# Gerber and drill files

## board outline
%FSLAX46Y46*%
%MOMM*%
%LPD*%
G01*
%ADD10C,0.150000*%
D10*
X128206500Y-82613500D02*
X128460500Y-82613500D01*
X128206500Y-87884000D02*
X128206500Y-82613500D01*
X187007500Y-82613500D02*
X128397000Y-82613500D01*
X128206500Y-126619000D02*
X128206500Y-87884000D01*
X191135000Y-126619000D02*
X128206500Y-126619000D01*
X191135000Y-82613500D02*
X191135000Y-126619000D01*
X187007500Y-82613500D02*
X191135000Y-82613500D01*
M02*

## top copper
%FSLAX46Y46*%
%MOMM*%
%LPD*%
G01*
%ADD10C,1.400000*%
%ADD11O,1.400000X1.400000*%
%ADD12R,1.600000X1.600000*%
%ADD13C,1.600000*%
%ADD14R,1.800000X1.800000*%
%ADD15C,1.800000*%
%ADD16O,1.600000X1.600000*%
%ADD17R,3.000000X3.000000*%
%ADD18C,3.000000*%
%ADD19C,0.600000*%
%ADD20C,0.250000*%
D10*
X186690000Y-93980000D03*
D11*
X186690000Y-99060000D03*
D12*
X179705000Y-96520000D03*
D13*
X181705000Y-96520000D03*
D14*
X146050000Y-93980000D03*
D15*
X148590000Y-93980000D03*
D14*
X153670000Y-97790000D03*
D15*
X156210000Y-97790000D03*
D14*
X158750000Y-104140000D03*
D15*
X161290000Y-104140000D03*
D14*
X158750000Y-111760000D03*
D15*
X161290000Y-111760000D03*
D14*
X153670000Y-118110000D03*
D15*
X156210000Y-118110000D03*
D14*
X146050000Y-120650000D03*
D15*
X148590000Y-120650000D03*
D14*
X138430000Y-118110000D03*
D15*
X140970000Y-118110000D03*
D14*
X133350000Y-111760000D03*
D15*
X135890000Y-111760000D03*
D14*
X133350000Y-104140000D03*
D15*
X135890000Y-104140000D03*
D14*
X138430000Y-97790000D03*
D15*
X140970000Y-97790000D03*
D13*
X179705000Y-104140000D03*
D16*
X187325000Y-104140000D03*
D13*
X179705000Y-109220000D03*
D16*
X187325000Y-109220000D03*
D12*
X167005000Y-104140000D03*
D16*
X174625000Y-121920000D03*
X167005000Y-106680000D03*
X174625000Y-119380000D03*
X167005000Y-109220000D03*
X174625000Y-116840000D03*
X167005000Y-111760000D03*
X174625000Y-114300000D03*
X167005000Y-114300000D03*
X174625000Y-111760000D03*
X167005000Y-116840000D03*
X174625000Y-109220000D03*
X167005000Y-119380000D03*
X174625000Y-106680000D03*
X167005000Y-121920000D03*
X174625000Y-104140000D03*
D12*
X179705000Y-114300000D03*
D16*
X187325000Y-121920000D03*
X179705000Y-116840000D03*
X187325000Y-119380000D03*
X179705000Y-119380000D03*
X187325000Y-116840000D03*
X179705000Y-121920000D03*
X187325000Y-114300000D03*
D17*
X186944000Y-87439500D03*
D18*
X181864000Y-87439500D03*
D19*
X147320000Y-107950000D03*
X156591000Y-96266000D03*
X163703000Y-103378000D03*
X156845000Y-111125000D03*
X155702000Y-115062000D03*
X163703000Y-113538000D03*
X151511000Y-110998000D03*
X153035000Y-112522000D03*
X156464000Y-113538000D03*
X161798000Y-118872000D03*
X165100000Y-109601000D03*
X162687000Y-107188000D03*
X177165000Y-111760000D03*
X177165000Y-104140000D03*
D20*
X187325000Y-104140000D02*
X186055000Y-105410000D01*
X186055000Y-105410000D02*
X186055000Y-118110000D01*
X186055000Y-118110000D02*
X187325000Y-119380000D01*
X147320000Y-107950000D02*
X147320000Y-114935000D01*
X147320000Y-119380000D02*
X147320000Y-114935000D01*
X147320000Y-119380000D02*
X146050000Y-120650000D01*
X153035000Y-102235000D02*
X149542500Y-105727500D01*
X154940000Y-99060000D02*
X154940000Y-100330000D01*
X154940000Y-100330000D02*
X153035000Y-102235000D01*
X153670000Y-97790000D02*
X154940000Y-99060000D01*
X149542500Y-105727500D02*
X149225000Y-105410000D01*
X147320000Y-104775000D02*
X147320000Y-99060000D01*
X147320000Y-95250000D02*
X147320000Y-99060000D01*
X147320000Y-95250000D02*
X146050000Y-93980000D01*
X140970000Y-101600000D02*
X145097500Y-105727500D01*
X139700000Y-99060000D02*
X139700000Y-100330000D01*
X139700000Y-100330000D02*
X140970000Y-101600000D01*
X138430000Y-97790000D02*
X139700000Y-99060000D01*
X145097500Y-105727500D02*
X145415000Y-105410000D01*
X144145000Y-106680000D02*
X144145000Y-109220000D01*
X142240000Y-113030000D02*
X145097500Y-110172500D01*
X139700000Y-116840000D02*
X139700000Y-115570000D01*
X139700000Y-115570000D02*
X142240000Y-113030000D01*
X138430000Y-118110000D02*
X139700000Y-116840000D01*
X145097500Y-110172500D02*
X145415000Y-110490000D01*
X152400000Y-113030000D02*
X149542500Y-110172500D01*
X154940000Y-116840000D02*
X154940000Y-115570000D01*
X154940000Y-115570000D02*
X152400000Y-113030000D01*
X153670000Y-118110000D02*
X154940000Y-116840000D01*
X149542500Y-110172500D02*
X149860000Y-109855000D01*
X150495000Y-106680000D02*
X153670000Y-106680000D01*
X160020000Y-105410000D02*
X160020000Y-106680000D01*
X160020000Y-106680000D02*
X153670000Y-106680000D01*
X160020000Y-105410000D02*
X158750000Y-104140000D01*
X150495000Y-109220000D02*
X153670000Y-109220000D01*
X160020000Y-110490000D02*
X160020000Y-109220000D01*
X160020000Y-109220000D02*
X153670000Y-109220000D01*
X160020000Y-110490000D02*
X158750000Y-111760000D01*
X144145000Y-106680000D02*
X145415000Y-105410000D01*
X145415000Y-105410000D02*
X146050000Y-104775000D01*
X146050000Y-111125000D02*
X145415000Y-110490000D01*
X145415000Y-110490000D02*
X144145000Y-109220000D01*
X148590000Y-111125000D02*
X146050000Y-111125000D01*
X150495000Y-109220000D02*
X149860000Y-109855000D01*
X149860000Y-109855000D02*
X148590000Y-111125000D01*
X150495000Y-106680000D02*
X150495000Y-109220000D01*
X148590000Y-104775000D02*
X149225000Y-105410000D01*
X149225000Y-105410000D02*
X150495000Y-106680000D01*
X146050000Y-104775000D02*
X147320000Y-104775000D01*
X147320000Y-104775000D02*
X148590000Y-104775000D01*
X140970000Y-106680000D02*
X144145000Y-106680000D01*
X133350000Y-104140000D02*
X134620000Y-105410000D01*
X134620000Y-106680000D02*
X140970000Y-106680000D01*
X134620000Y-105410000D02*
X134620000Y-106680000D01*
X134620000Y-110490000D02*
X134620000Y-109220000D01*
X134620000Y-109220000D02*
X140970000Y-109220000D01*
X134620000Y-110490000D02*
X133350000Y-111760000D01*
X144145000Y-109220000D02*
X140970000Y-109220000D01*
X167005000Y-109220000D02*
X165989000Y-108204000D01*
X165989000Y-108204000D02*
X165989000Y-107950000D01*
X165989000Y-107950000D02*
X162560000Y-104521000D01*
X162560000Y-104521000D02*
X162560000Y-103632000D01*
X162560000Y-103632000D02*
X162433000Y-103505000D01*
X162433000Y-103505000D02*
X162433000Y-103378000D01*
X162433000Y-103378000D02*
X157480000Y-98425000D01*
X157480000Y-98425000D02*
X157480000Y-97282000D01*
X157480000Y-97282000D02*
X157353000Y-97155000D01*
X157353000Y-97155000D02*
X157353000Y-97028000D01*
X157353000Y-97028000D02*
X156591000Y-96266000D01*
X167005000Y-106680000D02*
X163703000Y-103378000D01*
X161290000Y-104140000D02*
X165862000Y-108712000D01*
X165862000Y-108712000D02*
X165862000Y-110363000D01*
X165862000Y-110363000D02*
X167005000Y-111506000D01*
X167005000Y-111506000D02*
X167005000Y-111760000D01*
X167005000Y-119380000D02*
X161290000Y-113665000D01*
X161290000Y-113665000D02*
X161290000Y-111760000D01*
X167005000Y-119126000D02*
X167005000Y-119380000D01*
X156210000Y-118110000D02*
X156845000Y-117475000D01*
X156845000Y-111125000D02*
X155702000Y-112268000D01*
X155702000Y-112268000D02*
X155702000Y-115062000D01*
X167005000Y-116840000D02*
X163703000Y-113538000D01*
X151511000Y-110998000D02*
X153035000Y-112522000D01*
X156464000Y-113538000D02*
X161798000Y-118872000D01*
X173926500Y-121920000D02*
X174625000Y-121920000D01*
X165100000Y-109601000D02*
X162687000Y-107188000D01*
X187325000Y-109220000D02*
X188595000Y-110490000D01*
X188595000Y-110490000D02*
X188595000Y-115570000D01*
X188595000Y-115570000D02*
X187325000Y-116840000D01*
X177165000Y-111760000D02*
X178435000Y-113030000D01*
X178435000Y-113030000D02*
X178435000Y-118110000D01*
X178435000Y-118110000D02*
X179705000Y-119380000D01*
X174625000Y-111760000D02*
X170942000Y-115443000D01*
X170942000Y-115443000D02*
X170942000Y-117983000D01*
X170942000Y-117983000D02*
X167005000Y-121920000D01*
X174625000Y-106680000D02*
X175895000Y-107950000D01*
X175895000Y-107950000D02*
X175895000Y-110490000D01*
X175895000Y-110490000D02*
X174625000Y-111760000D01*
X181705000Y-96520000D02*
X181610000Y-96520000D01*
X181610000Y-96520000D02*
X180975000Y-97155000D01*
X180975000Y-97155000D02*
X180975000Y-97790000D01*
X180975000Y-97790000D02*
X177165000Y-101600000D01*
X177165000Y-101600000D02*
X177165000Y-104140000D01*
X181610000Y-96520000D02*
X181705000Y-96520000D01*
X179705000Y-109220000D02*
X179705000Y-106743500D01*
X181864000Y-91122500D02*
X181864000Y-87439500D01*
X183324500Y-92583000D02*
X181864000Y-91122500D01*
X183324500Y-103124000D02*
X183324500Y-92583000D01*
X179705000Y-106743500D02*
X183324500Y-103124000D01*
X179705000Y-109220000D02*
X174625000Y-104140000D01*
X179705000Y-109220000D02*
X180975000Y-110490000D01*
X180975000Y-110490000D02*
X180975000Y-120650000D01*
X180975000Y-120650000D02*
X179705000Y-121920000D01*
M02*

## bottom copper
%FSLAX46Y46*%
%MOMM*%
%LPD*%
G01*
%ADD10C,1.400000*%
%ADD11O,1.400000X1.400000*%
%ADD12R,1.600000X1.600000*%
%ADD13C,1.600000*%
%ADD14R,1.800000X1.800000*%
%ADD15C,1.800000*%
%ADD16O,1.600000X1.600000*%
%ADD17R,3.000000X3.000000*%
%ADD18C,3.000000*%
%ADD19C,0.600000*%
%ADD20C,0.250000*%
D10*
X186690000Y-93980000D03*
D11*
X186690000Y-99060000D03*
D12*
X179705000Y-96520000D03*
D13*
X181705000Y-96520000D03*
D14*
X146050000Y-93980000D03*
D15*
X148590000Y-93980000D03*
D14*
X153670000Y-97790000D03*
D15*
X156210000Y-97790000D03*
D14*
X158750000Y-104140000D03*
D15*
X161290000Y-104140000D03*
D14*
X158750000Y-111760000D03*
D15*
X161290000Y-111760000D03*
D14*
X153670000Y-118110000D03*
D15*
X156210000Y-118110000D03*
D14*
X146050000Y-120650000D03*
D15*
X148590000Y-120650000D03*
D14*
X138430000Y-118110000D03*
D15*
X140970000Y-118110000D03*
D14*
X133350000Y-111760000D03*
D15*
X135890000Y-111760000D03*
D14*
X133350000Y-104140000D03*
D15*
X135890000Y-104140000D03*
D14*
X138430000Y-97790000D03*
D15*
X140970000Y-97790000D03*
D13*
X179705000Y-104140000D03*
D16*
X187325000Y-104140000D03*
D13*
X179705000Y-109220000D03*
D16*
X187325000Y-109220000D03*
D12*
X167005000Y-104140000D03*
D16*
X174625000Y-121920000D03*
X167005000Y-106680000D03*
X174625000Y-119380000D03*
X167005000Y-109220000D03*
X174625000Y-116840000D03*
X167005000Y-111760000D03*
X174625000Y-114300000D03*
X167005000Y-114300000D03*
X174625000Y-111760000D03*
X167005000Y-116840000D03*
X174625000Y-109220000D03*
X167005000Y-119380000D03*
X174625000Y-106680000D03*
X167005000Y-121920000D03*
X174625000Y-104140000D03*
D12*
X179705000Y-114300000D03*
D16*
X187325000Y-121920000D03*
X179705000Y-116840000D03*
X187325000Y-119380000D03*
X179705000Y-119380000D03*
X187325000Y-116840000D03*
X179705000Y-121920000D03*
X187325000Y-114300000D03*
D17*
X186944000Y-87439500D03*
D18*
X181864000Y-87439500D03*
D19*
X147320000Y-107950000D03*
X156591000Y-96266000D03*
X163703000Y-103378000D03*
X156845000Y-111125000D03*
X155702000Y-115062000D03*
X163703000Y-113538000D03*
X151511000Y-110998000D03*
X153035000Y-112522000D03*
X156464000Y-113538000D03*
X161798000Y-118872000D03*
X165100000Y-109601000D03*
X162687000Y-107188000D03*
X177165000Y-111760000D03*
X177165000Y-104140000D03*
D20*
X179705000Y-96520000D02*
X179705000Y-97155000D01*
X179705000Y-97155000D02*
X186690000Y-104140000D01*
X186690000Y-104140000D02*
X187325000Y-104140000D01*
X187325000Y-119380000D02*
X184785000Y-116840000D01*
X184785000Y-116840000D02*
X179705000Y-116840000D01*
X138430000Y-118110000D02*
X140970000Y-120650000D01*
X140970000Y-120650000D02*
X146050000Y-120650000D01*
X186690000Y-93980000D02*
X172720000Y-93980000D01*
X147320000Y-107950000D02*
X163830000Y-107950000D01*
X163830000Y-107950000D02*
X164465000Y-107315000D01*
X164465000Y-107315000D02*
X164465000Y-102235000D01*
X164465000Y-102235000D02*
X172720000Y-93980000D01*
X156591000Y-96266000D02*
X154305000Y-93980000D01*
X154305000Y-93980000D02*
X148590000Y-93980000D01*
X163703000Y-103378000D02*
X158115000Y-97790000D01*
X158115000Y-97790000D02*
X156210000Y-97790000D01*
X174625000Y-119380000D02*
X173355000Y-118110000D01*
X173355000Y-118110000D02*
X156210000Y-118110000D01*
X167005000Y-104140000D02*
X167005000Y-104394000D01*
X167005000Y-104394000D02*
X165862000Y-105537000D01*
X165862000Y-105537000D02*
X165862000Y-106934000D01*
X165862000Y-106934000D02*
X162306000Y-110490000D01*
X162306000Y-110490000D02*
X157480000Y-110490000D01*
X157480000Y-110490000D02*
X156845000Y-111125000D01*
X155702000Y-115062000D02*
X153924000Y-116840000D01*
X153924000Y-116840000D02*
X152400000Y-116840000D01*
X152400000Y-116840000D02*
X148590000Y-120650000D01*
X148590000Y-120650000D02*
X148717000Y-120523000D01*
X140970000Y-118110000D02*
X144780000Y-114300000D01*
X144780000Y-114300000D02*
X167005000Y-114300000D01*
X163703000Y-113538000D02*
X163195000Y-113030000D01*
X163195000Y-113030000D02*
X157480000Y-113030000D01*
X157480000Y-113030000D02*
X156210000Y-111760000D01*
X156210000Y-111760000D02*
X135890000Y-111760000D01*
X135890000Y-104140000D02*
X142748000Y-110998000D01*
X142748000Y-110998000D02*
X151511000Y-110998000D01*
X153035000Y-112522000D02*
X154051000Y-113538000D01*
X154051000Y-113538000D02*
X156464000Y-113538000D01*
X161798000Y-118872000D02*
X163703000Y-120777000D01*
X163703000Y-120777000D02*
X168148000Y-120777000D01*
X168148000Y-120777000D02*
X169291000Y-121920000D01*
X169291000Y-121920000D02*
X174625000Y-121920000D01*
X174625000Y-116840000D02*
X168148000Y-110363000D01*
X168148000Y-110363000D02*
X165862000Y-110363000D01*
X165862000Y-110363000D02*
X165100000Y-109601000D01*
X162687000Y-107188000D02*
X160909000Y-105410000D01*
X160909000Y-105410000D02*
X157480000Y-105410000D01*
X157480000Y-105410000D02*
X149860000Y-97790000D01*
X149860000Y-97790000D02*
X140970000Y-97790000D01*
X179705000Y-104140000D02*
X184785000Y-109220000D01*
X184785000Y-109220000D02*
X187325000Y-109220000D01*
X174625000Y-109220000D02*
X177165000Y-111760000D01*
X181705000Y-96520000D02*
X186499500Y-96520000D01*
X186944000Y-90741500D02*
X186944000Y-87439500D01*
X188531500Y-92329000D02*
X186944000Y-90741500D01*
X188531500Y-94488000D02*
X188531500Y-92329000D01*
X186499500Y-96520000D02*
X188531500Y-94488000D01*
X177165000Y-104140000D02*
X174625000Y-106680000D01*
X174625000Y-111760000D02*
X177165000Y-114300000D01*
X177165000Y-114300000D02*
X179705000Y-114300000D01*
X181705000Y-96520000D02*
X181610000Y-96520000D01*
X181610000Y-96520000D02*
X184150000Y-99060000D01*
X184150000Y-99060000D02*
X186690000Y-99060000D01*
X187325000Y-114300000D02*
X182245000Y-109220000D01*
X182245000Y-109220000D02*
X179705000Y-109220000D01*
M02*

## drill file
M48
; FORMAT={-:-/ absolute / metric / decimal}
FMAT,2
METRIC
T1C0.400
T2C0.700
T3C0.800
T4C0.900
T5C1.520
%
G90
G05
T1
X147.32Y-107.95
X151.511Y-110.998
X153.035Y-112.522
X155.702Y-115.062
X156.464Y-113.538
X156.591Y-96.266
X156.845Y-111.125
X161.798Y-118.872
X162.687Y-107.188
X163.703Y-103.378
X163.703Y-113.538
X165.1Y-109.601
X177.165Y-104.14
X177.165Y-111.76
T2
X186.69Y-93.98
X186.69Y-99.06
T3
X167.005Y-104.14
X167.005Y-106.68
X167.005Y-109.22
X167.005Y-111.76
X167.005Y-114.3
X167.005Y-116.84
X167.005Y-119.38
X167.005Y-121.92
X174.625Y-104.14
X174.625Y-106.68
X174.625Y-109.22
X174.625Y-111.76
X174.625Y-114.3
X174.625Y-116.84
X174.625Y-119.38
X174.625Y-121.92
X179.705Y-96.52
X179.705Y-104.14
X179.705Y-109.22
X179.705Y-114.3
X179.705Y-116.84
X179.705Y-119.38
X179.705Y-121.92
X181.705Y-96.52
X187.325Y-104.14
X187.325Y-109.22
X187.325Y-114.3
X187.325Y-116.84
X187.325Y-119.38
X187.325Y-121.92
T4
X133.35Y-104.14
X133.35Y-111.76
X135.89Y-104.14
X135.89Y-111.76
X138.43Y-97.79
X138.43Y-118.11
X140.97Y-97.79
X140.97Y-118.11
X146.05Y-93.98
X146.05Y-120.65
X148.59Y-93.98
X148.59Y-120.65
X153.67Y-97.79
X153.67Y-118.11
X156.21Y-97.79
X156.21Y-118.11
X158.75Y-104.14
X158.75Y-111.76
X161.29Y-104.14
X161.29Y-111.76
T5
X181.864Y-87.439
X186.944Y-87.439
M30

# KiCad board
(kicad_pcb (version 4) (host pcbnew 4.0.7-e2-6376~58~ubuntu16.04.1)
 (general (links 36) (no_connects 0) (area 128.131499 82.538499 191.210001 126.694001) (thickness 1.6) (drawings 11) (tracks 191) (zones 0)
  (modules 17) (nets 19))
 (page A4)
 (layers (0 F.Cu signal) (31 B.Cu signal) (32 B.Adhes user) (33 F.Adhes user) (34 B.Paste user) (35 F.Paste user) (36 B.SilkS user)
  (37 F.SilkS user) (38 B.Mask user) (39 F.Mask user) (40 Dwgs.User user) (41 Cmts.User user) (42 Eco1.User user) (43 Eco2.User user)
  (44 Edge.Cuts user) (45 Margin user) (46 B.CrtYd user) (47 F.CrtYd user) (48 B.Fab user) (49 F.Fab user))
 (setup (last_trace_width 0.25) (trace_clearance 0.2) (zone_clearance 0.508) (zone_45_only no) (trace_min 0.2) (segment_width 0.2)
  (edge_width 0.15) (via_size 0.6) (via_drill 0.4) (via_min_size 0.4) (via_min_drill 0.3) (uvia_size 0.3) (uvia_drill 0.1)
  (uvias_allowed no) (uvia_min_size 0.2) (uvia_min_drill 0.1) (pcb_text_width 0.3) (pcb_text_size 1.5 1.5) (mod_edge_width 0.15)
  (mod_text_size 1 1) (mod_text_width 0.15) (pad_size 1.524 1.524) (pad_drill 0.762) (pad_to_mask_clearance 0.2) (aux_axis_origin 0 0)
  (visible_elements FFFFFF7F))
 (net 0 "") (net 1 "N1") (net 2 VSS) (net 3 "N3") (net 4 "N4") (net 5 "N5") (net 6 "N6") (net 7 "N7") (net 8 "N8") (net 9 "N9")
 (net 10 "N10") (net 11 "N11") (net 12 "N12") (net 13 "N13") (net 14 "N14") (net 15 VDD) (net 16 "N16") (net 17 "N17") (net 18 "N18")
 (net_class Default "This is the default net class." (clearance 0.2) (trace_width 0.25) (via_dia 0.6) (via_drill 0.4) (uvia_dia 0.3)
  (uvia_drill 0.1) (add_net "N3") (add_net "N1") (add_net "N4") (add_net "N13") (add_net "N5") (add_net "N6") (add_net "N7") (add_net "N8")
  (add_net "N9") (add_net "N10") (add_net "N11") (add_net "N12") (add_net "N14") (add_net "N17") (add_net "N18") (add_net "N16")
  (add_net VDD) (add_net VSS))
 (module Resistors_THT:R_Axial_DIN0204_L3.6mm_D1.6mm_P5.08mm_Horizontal (layer F.Cu) (at 186.69 93.98 270)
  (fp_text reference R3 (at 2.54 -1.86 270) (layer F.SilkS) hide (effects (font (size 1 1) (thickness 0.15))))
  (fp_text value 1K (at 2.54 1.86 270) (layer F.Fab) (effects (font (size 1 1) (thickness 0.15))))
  (pad 1 thru_hole circle (at 0 0 270) (size 1.4 1.4) (drill 0.7) (layers *.Cu *.Mask) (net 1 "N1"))
  (pad 2 thru_hole oval (at 5.08 0 270) (size 1.4 1.4) (drill 0.7) (layers *.Cu *.Mask) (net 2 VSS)))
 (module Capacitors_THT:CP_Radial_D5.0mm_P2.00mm (layer F.Cu) (at 179.705 96.52)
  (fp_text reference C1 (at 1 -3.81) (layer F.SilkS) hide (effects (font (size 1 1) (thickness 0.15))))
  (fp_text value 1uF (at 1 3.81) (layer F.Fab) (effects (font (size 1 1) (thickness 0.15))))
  (pad 1 thru_hole rect (at 0 0) (size 1.6 1.6) (drill 0.8) (layers *.Cu *.Mask) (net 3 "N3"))
  (pad 2 thru_hole circle (at 2 0) (size 1.6 1.6) (drill 0.8) (layers *.Cu *.Mask) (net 2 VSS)))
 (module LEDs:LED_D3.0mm (layer F.Cu) (at 146.05 93.98)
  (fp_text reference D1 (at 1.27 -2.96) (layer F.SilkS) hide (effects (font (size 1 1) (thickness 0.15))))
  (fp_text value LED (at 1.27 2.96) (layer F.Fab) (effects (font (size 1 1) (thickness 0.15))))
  (pad 1 thru_hole rect (at 0 0) (size 1.8 1.8) (drill 0.9) (layers *.Cu *.Mask) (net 1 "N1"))
  (pad 2 thru_hole circle (at 2.54 0) (size 1.8 1.8) (drill 0.9) (layers *.Cu *.Mask) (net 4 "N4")))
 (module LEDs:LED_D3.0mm (layer F.Cu) (at 153.67 97.79)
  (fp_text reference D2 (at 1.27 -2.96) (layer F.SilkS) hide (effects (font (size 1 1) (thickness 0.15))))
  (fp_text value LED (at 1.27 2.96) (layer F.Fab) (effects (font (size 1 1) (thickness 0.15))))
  (pad 1 thru_hole rect (at 0 0) (size 1.8 1.8) (drill 0.9) (layers *.Cu *.Mask) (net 1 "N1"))
  (pad 2 thru_hole circle (at 2.54 0) (size 1.8 1.8) (drill 0.9) (layers *.Cu *.Mask) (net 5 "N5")))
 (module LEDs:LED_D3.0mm (layer F.Cu) (at 158.75 104.14)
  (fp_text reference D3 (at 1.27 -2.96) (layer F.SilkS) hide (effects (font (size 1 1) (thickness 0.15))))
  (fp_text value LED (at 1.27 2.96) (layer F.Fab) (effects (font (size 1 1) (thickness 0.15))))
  (pad 1 thru_hole rect (at 0 0) (size 1.8 1.8) (drill 0.9) (layers *.Cu *.Mask) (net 1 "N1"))
  (pad 2 thru_hole circle (at 2.54 0) (size 1.8 1.8) (drill 0.9) (layers *.Cu *.Mask) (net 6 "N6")))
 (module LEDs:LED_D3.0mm (layer F.Cu) (at 158.75 111.76)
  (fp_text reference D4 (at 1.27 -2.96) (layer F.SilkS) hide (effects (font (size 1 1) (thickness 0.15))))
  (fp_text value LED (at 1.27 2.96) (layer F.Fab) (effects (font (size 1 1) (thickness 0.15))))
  (pad 1 thru_hole rect (at 0 0) (size 1.8 1.8) (drill 0.9) (layers *.Cu *.Mask) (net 1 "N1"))
  (pad 2 thru_hole circle (at 2.54 0) (size 1.8 1.8) (drill 0.9) (layers *.Cu *.Mask) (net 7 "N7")))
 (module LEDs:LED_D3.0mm (layer F.Cu) (at 153.67 118.11)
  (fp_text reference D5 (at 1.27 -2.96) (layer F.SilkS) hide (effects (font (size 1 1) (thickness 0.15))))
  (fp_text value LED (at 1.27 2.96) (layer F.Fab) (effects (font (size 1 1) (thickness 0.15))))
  (pad 1 thru_hole rect (at 0 0) (size 1.8 1.8) (drill 0.9) (layers *.Cu *.Mask) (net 1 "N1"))
  (pad 2 thru_hole circle (at 2.54 0) (size 1.8 1.8) (drill 0.9) (layers *.Cu *.Mask) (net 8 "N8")))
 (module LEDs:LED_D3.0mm (layer F.Cu) (at 146.05 120.65)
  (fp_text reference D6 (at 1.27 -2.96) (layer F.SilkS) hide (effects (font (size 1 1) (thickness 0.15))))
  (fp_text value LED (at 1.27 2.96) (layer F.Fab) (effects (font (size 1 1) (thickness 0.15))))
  (pad 1 thru_hole rect (at 0 0) (size 1.8 1.8) (drill 0.9) (layers *.Cu *.Mask) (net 1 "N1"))
  (pad 2 thru_hole circle (at 2.54 0) (size 1.8 1.8) (drill 0.9) (layers *.Cu *.Mask) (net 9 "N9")))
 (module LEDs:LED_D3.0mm (layer F.Cu) (at 138.43 118.11)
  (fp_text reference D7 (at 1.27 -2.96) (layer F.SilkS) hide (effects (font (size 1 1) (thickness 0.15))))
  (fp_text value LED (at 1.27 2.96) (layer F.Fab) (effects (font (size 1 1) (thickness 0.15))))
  (pad 1 thru_hole rect (at 0 0) (size 1.8 1.8) (drill 0.9) (layers *.Cu *.Mask) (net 1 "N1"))
  (pad 2 thru_hole circle (at 2.54 0) (size 1.8 1.8) (drill 0.9) (layers *.Cu *.Mask) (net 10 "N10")))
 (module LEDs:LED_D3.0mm (layer F.Cu) (at 133.35 111.76)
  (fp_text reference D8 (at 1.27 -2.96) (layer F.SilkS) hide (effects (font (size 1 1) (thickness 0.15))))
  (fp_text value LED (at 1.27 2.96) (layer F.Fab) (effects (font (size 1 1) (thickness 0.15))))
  (pad 1 thru_hole rect (at 0 0) (size 1.8 1.8) (drill 0.9) (layers *.Cu *.Mask) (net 1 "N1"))
  (pad 2 thru_hole circle (at 2.54 0) (size 1.8 1.8) (drill 0.9) (layers *.Cu *.Mask) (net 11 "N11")))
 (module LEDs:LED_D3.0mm (layer F.Cu) (at 133.35 104.14)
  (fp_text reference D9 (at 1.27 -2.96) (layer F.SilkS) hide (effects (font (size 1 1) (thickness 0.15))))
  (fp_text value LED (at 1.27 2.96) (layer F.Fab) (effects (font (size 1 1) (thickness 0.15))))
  (pad 1 thru_hole rect (at 0 0) (size 1.8 1.8) (drill 0.9) (layers *.Cu *.Mask) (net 1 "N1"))
  (pad 2 thru_hole circle (at 2.54 0) (size 1.8 1.8) (drill 0.9) (layers *.Cu *.Mask) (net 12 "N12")))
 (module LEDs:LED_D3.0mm (layer F.Cu) (at 138.43 97.79)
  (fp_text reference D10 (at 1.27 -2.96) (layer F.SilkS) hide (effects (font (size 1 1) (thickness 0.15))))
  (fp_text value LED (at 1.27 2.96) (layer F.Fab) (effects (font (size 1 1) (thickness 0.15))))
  (pad 1 thru_hole rect (at 0 0) (size 1.8 1.8) (drill 0.9) (layers *.Cu *.Mask) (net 1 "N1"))
  (pad 2 thru_hole circle (at 2.54 0) (size 1.8 1.8) (drill 0.9) (layers *.Cu *.Mask) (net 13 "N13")))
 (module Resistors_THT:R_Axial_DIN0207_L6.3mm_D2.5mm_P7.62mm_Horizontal (layer F.Cu) (at 179.705 104.14)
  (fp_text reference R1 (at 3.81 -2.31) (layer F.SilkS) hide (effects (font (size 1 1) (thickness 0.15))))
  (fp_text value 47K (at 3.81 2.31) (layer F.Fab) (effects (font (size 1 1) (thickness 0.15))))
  (pad 1 thru_hole circle (at 0 0) (size 1.6 1.6) (drill 0.8) (layers *.Cu *.Mask) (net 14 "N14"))
  (pad 2 thru_hole oval (at 7.62 0) (size 1.6 1.6) (drill 0.8) (layers *.Cu *.Mask) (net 3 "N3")))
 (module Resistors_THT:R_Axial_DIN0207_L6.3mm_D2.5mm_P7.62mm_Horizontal (layer F.Cu) (at 179.705 109.22)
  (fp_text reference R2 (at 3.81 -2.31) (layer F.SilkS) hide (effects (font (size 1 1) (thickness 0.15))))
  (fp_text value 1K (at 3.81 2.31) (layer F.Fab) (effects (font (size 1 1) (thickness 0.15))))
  (pad 1 thru_hole circle (at 0 0) (size 1.6 1.6) (drill 0.8) (layers *.Cu *.Mask) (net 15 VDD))
  (pad 2 thru_hole oval (at 7.62 0) (size 1.6 1.6) (drill 0.8) (layers *.Cu *.Mask) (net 14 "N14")))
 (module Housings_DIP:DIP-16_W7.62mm (layer F.Cu) (at 167.005 104.14)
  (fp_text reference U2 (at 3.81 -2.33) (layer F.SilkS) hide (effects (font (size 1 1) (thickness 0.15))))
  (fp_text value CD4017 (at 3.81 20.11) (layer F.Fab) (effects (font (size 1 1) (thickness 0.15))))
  (pad 1 thru_hole rect (at 0 0) (size 1.6 1.6) (drill 0.8) (layers *.Cu *.Mask) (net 9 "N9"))
  (pad 9 thru_hole oval (at 7.62 17.78) (size 1.6 1.6) (drill 0.8) (layers *.Cu *.Mask) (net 12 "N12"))
  (pad 2 thru_hole oval (at 0 2.54) (size 1.6 1.6) (drill 0.8) (layers *.Cu *.Mask) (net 5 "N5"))
  (pad 10 thru_hole oval (at 7.62 15.24) (size 1.6 1.6) (drill 0.8) (layers *.Cu *.Mask) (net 8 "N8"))
  (pad 3 thru_hole oval (at 0 5.08) (size 1.6 1.6) (drill 0.8) (layers *.Cu *.Mask) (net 4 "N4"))
  (pad 11 thru_hole oval (at 7.62 12.7) (size 1.6 1.6) (drill 0.8) (layers *.Cu *.Mask) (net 13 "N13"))
  (pad 4 thru_hole oval (at 0 7.62) (size 1.6 1.6) (drill 0.8) (layers *.Cu *.Mask) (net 6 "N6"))
  (pad 12 thru_hole oval (at 7.62 10.16) (size 1.6 1.6) (drill 0.8) (layers *.Cu *.Mask) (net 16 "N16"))
  (pad 5 thru_hole oval (at 0 10.16) (size 1.6 1.6) (drill 0.8) (layers *.Cu *.Mask) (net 10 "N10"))
  (pad 13 thru_hole oval (at 7.62 7.62) (size 1.6 1.6) (drill 0.8) (layers *.Cu *.Mask) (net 2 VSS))
  (pad 6 thru_hole oval (at 0 12.7) (size 1.6 1.6) (drill 0.8) (layers *.Cu *.Mask) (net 11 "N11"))
  (pad 14 thru_hole oval (at 7.62 5.08) (size 1.6 1.6) (drill 0.8) (layers *.Cu *.Mask) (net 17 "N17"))
  (pad 7 thru_hole oval (at 0 15.24) (size 1.6 1.6) (drill 0.8) (layers *.Cu *.Mask) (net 7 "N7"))
  (pad 15 thru_hole oval (at 7.62 2.54) (size 1.6 1.6) (drill 0.8) (layers *.Cu *.Mask) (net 2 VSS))
  (pad 8 thru_hole oval (at 0 17.78) (size 1.6 1.6) (drill 0.8) (layers *.Cu *.Mask) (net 2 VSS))
  (pad 16 thru_hole oval (at 7.62 0) (size 1.6 1.6) (drill 0.8) (layers *.Cu *.Mask) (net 15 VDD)))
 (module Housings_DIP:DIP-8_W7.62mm (layer F.Cu) (at 179.705 114.3)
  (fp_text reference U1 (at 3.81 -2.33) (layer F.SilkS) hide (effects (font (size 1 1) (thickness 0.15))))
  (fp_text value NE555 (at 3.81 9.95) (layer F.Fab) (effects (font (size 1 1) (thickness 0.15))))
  (pad 1 thru_hole rect (at 0 0) (size 1.6 1.6) (drill 0.8) (layers *.Cu *.Mask) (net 2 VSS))
  (pad 5 thru_hole oval (at 7.62 7.62) (size 1.6 1.6) (drill 0.8) (layers *.Cu *.Mask) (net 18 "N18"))
  (pad 2 thru_hole oval (at 0 2.54) (size 1.6 1.6) (drill 0.8) (layers *.Cu *.Mask) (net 3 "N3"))
  (pad 6 thru_hole oval (at 7.62 5.08) (size 1.6 1.6) (drill 0.8) (layers *.Cu *.Mask) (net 3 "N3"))
  (pad 3 thru_hole oval (at 0 5.08) (size 1.6 1.6) (drill 0.8) (layers *.Cu *.Mask) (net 17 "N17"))
  (pad 7 thru_hole oval (at 7.62 2.54) (size 1.6 1.6) (drill 0.8) (layers *.Cu *.Mask) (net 14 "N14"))
  (pad 4 thru_hole oval (at 0 7.62) (size 1.6 1.6) (drill 0.8) (layers *.Cu *.Mask) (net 15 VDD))
  (pad 8 thru_hole oval (at 7.62 0) (size 1.6 1.6) (drill 0.8) (layers *.Cu *.Mask) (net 15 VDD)))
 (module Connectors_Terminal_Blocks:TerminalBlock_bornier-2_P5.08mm (layer F.Cu) (at 186.944 87.4395 180)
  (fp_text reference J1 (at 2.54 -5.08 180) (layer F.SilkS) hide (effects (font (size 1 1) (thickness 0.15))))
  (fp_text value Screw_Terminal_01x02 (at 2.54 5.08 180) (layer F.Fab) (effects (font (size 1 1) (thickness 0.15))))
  (pad 1 thru_hole rect (at 0 0 180) (size 3 3) (drill 1.52) (layers *.Cu *.Mask) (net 2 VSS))
  (pad 2 thru_hole circle (at 5.08 0 180) (size 3 3) (drill 1.52) (layers *.Cu *.Mask) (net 15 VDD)))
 (gr_line (start 128.2065 82.6135) (end 128.4605 82.6135) (angle 90) (layer Edge.Cuts) (width 0.15))
 (gr_line (start 128.2065 87.884) (end 128.2065 82.6135) (angle 90) (layer Edge.Cuts) (width 0.15))
 (gr_line (start 187.0075 82.6135) (end 128.397 82.6135) (angle 90) (layer Edge.Cuts) (width 0.15))
 (gr_line (start 128.2065 126.619) (end 128.2065 87.884) (angle 90) (layer Edge.Cuts) (width 0.15))
 (gr_line (start 191.135 126.619) (end 128.2065 126.619) (angle 90) (layer Edge.Cuts) (width 0.15))
 (gr_line (start 191.135 82.6135) (end 191.135 126.619) (angle 90) (layer Edge.Cuts) (width 0.15))
 (gr_line (start 187.0075 82.6135) (end 191.135 82.6135) (angle 90) (layer Edge.Cuts) (width 0.15))
 (segment (start 179.705 96.52) (end 179.705 97.155) (width 0.25) (layer B.Cu) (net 3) (status 80000))
 (segment (start 179.705 97.155) (end 186.69 104.14) (width 0.25) (layer B.Cu) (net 3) (status 80000))
 (segment (start 186.69 104.14) (end 187.325 104.14) (width 0.25) (layer B.Cu) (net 3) (status 80000))
 (segment (start 187.325 119.38) (end 184.785 116.84) (width 0.25) (layer B.Cu) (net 3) (status 80000))
 (segment (start 184.785 116.84) (end 179.705 116.84) (width 0.25) (layer B.Cu) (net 3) (status 80000))
 (segment (start 187.325 104.14) (end 186.055 105.41) (width 0.25) (layer F.Cu) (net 3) (status 80000))
 (segment (start 186.055 105.41) (end 186.055 118.11) (width 0.25) (layer F.Cu) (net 3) (status 80000))
 (segment (start 186.055 118.11) (end 187.325 119.38) (width 0.25) (layer F.Cu) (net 3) (status 80000))
 (segment (start 138.43 118.11) (end 140.97 120.65) (width 0.25) (layer B.Cu) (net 1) (status 80000))
 (segment (start 140.97 120.65) (end 146.05 120.65) (width 0.25) (layer B.Cu) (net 1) (status 80000))
 (segment (start 186.69 93.98) (end 172.72 93.98) (width 0.25) (layer B.Cu) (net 1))
 (segment (start 147.32 107.95) (end 163.83 107.95) (width 0.25) (layer B.Cu) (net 1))
 (segment (start 163.83 107.95) (end 164.465 107.315) (width 0.25) (layer B.Cu) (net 1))
 (segment (start 164.465 107.315) (end 164.465 102.235) (width 0.25) (layer B.Cu) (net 1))
 (segment (start 164.465 102.235) (end 172.72 93.98) (width 0.25) (layer B.Cu) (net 1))
 (segment (start 147.32 107.95) (end 147.32 114.935) (width 0.25) (layer F.Cu) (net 1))
 (segment (start 147.32 119.38) (end 147.32 114.935) (width 0.25) (layer F.Cu) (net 1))
 (segment (start 147.32 119.38) (end 146.05 120.65) (width 0.25) (layer F.Cu) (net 1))
 (via (at 147.32 107.95) (size 0.6) (drill 0.4) (layers F.Cu B.Cu) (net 1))
 (segment (start 153.035 102.235) (end 149.5425 105.7275) (width 0.25) (layer F.Cu) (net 1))
 (segment (start 154.94 99.06) (end 154.94 100.33) (width 0.25) (layer F.Cu) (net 1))
 (segment (start 154.94 100.33) (end 153.035 102.235) (width 0.25) (layer F.Cu) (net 1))
 (segment (start 153.67 97.79) (end 154.94 99.06) (width 0.25) (layer F.Cu) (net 1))
 (segment (start 149.5425 105.7275) (end 149.225 105.41) (width 0.25) (layer F.Cu) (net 1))
 (segment (start 147.32 104.775) (end 147.32 99.06) (width 0.25) (layer F.Cu) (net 1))
 (segment (start 147.32 95.25) (end 147.32 99.06) (width 0.25) (layer F.Cu) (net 1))
 (segment (start 147.32 95.25) (end 146.05 93.98) (width 0.25) (layer F.Cu) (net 1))
 (segment (start 140.97 101.6) (end 145.0975 105.7275) (width 0.25) (layer F.Cu) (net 1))
 (segment (start 139.7 99.06) (end 139.7 100.33) (width 0.25) (layer F.Cu) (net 1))
 (segment (start 139.7 100.33) (end 140.97 101.6) (width 0.25) (layer F.Cu) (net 1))
 (segment (start 138.43 97.79) (end 139.7 99.06) (width 0.25) (layer F.Cu) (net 1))
 (segment (start 145.0975 105.7275) (end 145.415 105.41) (width 0.25) (layer F.Cu) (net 1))
 (segment (start 144.145 106.68) (end 144.145 109.22) (width 0.25) (layer F.Cu) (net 1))
 (segment (start 142.24 113.03) (end 145.0975 110.1725) (width 0.25) (layer F.Cu) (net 1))
 (segment (start 139.7 116.84) (end 139.7 115.57) (width 0.25) (layer F.Cu) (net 1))
 (segment (start 139.7 115.57) (end 142.24 113.03) (width 0.25) (layer F.Cu) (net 1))
 (segment (start 138.43 118.11) (end 139.7 116.84) (width 0.25) (layer F.Cu) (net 1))
 (segment (start 145.0975 110.1725) (end 145.415 110.49) (width 0.25) (layer F.Cu) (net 1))
 (segment (start 152.4 113.03) (end 149.5425 110.1725) (width 0.25) (layer F.Cu) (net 1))
 (segment (start 154.94 116.84) (end 154.94 115.57) (width 0.25) (layer F.Cu) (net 1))
 (segment (start 154.94 115.57) (end 152.4 113.03) (width 0.25) (layer F.Cu) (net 1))
 (segment (start 153.67 118.11) (end 154.94 116.84) (width 0.25) (layer F.Cu) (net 1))
 (segment (start 149.5425 110.1725) (end 149.86 109.855) (width 0.25) (layer F.Cu) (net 1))
 (segment (start 150.495 106.68) (end 153.67 106.68) (width 0.25) (layer F.Cu) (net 1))
 (segment (start 160.02 105.41) (end 160.02 106.68) (width 0.25) (layer F.Cu) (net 1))
 (segment (start 160.02 106.68) (end 153.67 106.68) (width 0.25) (layer F.Cu) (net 1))
 (segment (start 160.02 105.41) (end 158.75 104.14) (width 0.25) (layer F.Cu) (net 1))
 (segment (start 150.495 109.22) (end 153.67 109.22) (width 0.25) (layer F.Cu) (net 1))
 (segment (start 160.02 110.49) (end 160.02 109.22) (width 0.25) (layer F.Cu) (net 1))
 (segment (start 160.02 109.22) (end 153.67 109.22) (width 0.25) (layer F.Cu) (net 1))
 (segment (start 160.02 110.49) (end 158.75 111.76) (width 0.25) (layer F.Cu) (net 1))
 (segment (start 144.145 106.68) (end 145.415 105.41) (width 0.25) (layer F.Cu) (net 1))
 (segment (start 145.415 105.41) (end 146.05 104.775) (width 0.25) (layer F.Cu) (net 1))
 (segment (start 146.05 111.125) (end 145.415 110.49) (width 0.25) (layer F.Cu) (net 1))
 (segment (start 145.415 110.49) (end 144.145 109.22) (width 0.25) (layer F.Cu) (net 1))
 (segment (start 148.59 111.125) (end 146.05 111.125) (width 0.25) (layer F.Cu) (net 1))
 (segment (start 150.495 109.22) (end 149.86 109.855) (width 0.25) (layer F.Cu) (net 1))
 (segment (start 149.86 109.855) (end 148.59 111.125) (width 0.25) (layer F.Cu) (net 1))
 (segment (start 150.495 106.68) (end 150.495 109.22) (width 0.25) (layer F.Cu) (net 1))
 (segment (start 148.59 104.775) (end 149.225 105.41) (width 0.25) (layer F.Cu) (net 1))
 (segment (start 149.225 105.41) (end 150.495 106.68) (width 0.25) (layer F.Cu) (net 1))
 (segment (start 146.05 104.775) (end 147.32 104.775) (width 0.25) (layer F.Cu) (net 1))
 (segment (start 147.32 104.775) (end 148.59 104.775) (width 0.25) (layer F.Cu) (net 1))
 (segment (start 140.97 106.68) (end 144.145 106.68) (width 0.25) (layer F.Cu) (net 1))
 (segment (start 133.35 104.14) (end 134.62 105.41) (width 0.25) (layer F.Cu) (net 1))
 (segment (start 134.62 106.68) (end 140.97 106.68) (width 0.25) (layer F.Cu) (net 1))
 (segment (start 134.62 105.41) (end 134.62 106.68) (width 0.25) (layer F.Cu) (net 1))
 (segment (start 134.62 110.49) (end 134.62 109.22) (width 0.25) (layer F.Cu) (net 1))
 (segment (start 134.62 109.22) (end 140.97 109.22) (width 0.25) (layer F.Cu) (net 1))
 (segment (start 134.62 110.49) (end 133.35 111.76) (width 0.25) (layer F.Cu) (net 1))
 (segment (start 144.145 109.22) (end 140.97 109.22) (width 0.25) (layer F.Cu) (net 1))
 (segment (start 167.005 109.22) (end 165.989 108.204) (width 0.25) (layer F.Cu) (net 4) (status 80000))
 (segment (start 165.989 108.204) (end 165.989 107.95) (width 0.25) (layer F.Cu) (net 4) (status 80000))
 (segment (start 165.989 107.95) (end 162.56 104.521) (width 0.25) (layer F.Cu) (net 4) (status 80000))
 (segment (start 162.56 104.521) (end 162.56 103.632) (width 0.25) (layer F.Cu) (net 4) (status 80000))
 (segment (start 162.56 103.632) (end 162.433 103.505) (width 0.25) (layer F.Cu) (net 4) (status 80000))
 (segment (start 162.433 103.505) (end 162.433 103.378) (width 0.25) (layer F.Cu) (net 4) (status 80000))
 (segment (start 162.433 103.378) (end 157.48 98.425) (width 0.25) (layer F.Cu) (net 4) (status 80000))
 (segment (start 157.48 98.425) (end 157.48 97.282) (width 0.25) (layer F.Cu) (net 4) (status 80000))
 (segment (start 157.48 97.282) (end 157.353 97.155) (width 0.25) (layer F.Cu) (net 4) (status 80000))
 (segment (start 157.353 97.155) (end 157.353 97.028) (width 0.25) (layer F.Cu) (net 4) (status 80000))
 (segment (start 157.353 97.028) (end 156.591 96.266) (width 0.25) (layer F.Cu) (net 4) (status 80000))
 (via (at 156.591 96.266) (size 0.6) (layers F.Cu B.Cu) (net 4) (status 80000))
 (segment (start 156.591 96.266) (end 154.305 93.98) (width 0.25) (layer B.Cu) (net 4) (status 80000))
 (segment (start 154.305 93.98) (end 148.59 93.98) (width 0.25) (layer B.Cu) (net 4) (status 80000))
 (segment (start 167.005 106.68) (end 163.703 103.378) (width 0.25) (layer F.Cu) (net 5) (status 80000))
 (via (at 163.703 103.378) (size 0.6) (layers F.Cu B.Cu) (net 5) (status 80000))
 (segment (start 163.703 103.378) (end 158.115 97.79) (width 0.25) (layer B.Cu) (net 5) (status 80000))
 (segment (start 158.115 97.79) (end 156.21 97.79) (width 0.25) (layer B.Cu) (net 5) (status 80000))
 (segment (start 161.29 104.14) (end 165.862 108.712) (width 0.25) (layer F.Cu) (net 6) (status 80000))
 (segment (start 165.862 108.712) (end 165.862 110.363) (width 0.25) (layer F.Cu) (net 6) (status 80000))
 (segment (start 165.862 110.363) (end 167.005 111.506) (width 0.25) (layer F.Cu) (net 6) (status 80000))
 (segment (start 167.005 111.506) (end 167.005 111.76) (width 0.25) (layer F.Cu) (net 6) (status 80000))
 (segment (start 167.005 119.38) (end 161.29 113.665) (width 0.25) (layer F.Cu) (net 7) (status 80000))
 (segment (start 161.29 113.665) (end 161.29 111.76) (width 0.25) (layer F.Cu) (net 7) (status 80000))
 (segment (start 167.005 119.126) (end 167.005 119.38) (width 0.25) (layer F.Cu) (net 7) (status 80000))
 (segment (start 174.625 119.38) (end 173.355 118.11) (width 0.25) (layer B.Cu) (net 8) (status 80000))
 (segment (start 173.355 118.11) (end 156.21 118.11) (width 0.25) (layer B.Cu) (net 8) (status 80000))
 (segment (start 156.21 118.11) (end 156.845 117.475) (width 0.25) (layer F.Cu) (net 8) (status 80000))
 (segment (start 167.005 104.14) (end 167.005 104.394) (width 0.25) (layer B.Cu) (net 9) (status 80000))
 (segment (start 167.005 104.394) (end 165.862 105.537) (width 0.25) (layer B.Cu) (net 9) (status 80000))
 (segment (start 165.862 105.537) (end 165.862 106.934) (width 0.25) (layer B.Cu) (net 9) (status 80000))
 (segment (start 165.862 106.934) (end 162.306 110.49) (width 0.25) (layer B.Cu) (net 9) (status 80000))
 (segment (start 162.306 110.49) (end 157.48 110.49) (width 0.25) (layer B.Cu) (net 9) (status 80000))
 (segment (start 157.48 110.49) (end 156.845 111.125) (width 0.25) (layer B.Cu) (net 9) (status 80000))
 (via (at 156.845 111.125) (size 0.6) (layers F.Cu B.Cu) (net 9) (status 80000))
 (segment (start 156.845 111.125) (end 155.702 112.268) (width 0.25) (layer F.Cu) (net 9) (status 80000))
 (segment (start 155.702 112.268) (end 155.702 115.062) (width 0.25) (layer F.Cu) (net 9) (status 80000))
 (via (at 155.702 115.062) (size 0.6) (layers F.Cu B.Cu) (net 9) (status 80000))
 (segment (start 155.702 115.062) (end 153.924 116.84) (width 0.25) (layer B.Cu) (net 9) (status 80000))
 (segment (start 153.924 116.84) (end 152.4 116.84) (width 0.25) (layer B.Cu) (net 9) (status 80000))
 (segment (start 152.4 116.84) (end 148.59 120.65) (width 0.25) (layer B.Cu) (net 9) (status 80000))
 (segment (start 148.59 120.65) (end 148.717 120.523) (width 0.25) (layer B.Cu) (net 9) (status 80000))
 (segment (start 140.97 118.11) (end 144.78 114.3) (width 0.25) (layer B.Cu) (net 10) (status 80000))
 (segment (start 144.78 114.3) (end 167.005 114.3) (width 0.25) (layer B.Cu) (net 10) (status 80000))
 (segment (start 167.005 116.84) (end 163.703 113.538) (width 0.25) (layer F.Cu) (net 11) (status 80000))
 (via (at 163.703 113.538) (size 0.6) (layers F.Cu B.Cu) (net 11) (status 80000))
 (segment (start 163.703 113.538) (end 163.195 113.03) (width 0.25) (layer B.Cu) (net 11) (status 80000))
 (segment (start 163.195 113.03) (end 157.48 113.03) (width 0.25) (layer B.Cu) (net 11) (status 80000))
 (segment (start 157.48 113.03) (end 156.21 111.76) (width 0.25) (layer B.Cu) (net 11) (status 80000))
 (segment (start 156.21 111.76) (end 135.89 111.76) (width 0.25) (layer B.Cu) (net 11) (status 80000))
 (segment (start 135.89 104.14) (end 142.748 110.998) (width 0.25) (layer B.Cu) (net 12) (status 80000))
 (segment (start 142.748 110.998) (end 151.511 110.998) (width 0.25) (layer B.Cu) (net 12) (status 80000))
 (via (at 151.511 110.998) (size 0.6) (layers F.Cu B.Cu) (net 12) (status 80000))
 (segment (start 151.511 110.998) (end 153.035 112.522) (width 0.25) (layer F.Cu) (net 12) (status 80000))
 (via (at 153.035 112.522) (size 0.6) (layers F.Cu B.Cu) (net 12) (status 80000))
 (segment (start 153.035 112.522) (end 154.051 113.538) (width 0.25) (layer B.Cu) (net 12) (status 80000))
 (segment (start 154.051 113.538) (end 156.464 113.538) (width 0.25) (layer B.Cu) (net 12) (status 80000))
 (via (at 156.464 113.538) (size 0.6) (layers F.Cu B.Cu) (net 12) (status 80000))
 (segment (start 156.464 113.538) (end 161.798 118.872) (width 0.25) (layer F.Cu) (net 12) (status 80000))
 (via (at 161.798 118.872) (size 0.6) (layers F.Cu B.Cu) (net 12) (status 80000))
 (segment (start 161.798 118.872) (end 163.703 120.777) (width 0.25) (layer B.Cu) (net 12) (status 80000))
 (segment (start 163.703 120.777) (end 168.148 120.777) (width 0.25) (layer B.Cu) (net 12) (status 80000))
 (segment (start 168.148 120.777) (end 169.291 121.92) (width 0.25) (layer B.Cu) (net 12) (status 80000))
 (segment (start 169.291 121.92) (end 174.625 121.92) (width 0.25) (layer B.Cu) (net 12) (status 80000))
 (segment (start 173.9265 121.92) (end 174.625 121.92) (width 0.25) (layer F.Cu) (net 12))
 (segment (start 174.625 116.84) (end 168.148 110.363) (width 0.25) (layer B.Cu) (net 13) (status 80000))
 (segment (start 168.148 110.363) (end 165.862 110.363) (width 0.25) (layer B.Cu) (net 13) (status 80000))
 (segment (start 165.862 110.363) (end 165.1 109.601) (width 0.25) (layer B.Cu) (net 13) (status 80000))
 (via (at 165.1 109.601) (size 0.6) (layers F.Cu B.Cu) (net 13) (status 80000))
 (segment (start 165.1 109.601) (end 162.687 107.188) (width 0.25) (layer F.Cu) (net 13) (status 80000))
 (via (at 162.687 107.188) (size 0.6) (layers F.Cu B.Cu) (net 13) (status 80000))
 (segment (start 162.687 107.188) (end 160.909 105.41) (width 0.25) (layer B.Cu) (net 13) (status 80000))
 (segment (start 160.909 105.41) (end 157.48 105.41) (width 0.25) (layer B.Cu) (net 13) (status 80000))
 (segment (start 157.48 105.41) (end 149.86 97.79) (width 0.25) (layer B.Cu) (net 13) (status 80000))
 (segment (start 149.86 97.79) (end 140.97 97.79) (width 0.25) (layer B.Cu) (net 13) (status 80000))
 (segment (start 179.705 104.14) (end 184.785 109.22) (width 0.25) (layer B.Cu) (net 14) (status 80000))
 (segment (start 184.785 109.22) (end 187.325 109.22) (width 0.25) (layer B.Cu) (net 14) (status 80000))
 (segment (start 187.325 109.22) (end 188.595 110.49) (width 0.25) (layer F.Cu) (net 14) (status 80000))
 (segment (start 188.595 110.49) (end 188.595 115.57) (width 0.25) (layer F.Cu) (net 14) (status 80000))
 (segment (start 188.595 115.57) (end 187.325 116.84) (width 0.25) (layer F.Cu) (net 14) (status 80000))
 (segment (start 174.625 109.22) (end 177.165 111.76) (width 0.25) (layer B.Cu) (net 17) (status 80000))
 (via (at 177.165 111.76) (size 0.6) (layers F.Cu B.Cu) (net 17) (status 80000))
 (segment (start 177.165 111.76) (end 178.435 113.03) (width 0.25) (layer F.Cu) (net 17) (status 80000))
 (segment (start 178.435 113.03) (end 178.435 118.11) (width 0.25) (layer F.Cu) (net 17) (status 80000))
 (segment (start 178.435 118.11) (end 179.705 119.38) (width 0.25) (layer F.Cu) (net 17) (status 80000))
 (segment (start 181.705 96.52) (end 186.4995 96.52) (width 0.25) (layer B.Cu) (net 2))
 (segment (start 186.944 90.7415) (end 186.944 87.4395) (width 0.25) (layer B.Cu) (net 2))
 (segment (start 188.5315 92.329) (end 186.944 90.7415) (width 0.25) (layer B.Cu) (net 2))
 (segment (start 188.5315 94.488) (end 188.5315 92.329) (width 0.25) (layer B.Cu) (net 2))
 (segment (start 186.4995 96.52) (end 188.5315 94.488) (width 0.25) (layer B.Cu) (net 2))
 (segment (start 174.625 111.76) (end 170.942 115.443) (width 0.25) (layer F.Cu) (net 2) (status 80000))
 (segment (start 170.942 115.443) (end 170.942 117.983) (width 0.25) (layer F.Cu) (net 2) (status 80000))
 (segment (start 170.942 117.983) (end 167.005 121.92) (width 0.25) (layer F.Cu) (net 2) (status 80000))
 (segment (start 174.625 106.68) (end 175.895 107.95) (width 0.25) (layer F.Cu) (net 2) (status 80000))
 (segment (start 175.895 107.95) (end 175.895 110.49) (width 0.25) (layer F.Cu) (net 2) (status 80000))
 (segment (start 175.895 110.49) (end 174.625 111.76) (width 0.25) (layer F.Cu) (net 2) (status 80000))
 (segment (start 181.705 96.52) (end 181.61 96.52) (width 0.25) (layer F.Cu) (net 2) (status 80000))
 (segment (start 181.61 96.52) (end 180.975 97.155) (width 0.25) (layer F.Cu) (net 2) (status 80000))
 (segment (start 180.975 97.155) (end 180.975 97.79) (width 0.25) (layer F.Cu) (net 2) (status 80000))
 (segment (start 180.975 97.79) (end 177.165 101.6) (width 0.25) (layer F.Cu) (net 2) (status 80000))
 (segment (start 177.165 101.6) (end 177.165 104.14) (width 0.25) (layer F.Cu) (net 2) (status 80000))
 (via (at 177.165 104.14) (size 0.6) (layers F.Cu B.Cu) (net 2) (status 80000))
 (segment (start 177.165 104.14) (end 174.625 106.68) (width 0.25) (layer B.Cu) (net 2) (status 80000))
 (segment (start 174.625 111.76) (end 177.165 114.3) (width 0.25) (layer B.Cu) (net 2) (status 80000))
 (segment (start 177.165 114.3) (end 179.705 114.3) (width 0.25) (layer B.Cu) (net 2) (status 80000))
 (segment (start 181.705 96.52) (end 181.61 96.52) (width 0.25) (layer B.Cu) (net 2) (status 80000))
 (segment (start 181.61 96.52) (end 184.15 99.06) (width 0.25) (layer B.Cu) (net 2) (status 80000))
 (segment (start 184.15 99.06) (end 186.69 99.06) (width 0.25) (layer B.Cu) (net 2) (status 80000))
 (segment (start 181.61 96.52) (end 181.705 96.52) (width 0.25) (layer F.Cu) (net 2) (status 80000))
 (segment (start 179.705 109.22) (end 179.705 106.7435) (width 0.25) (layer F.Cu) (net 15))
 (segment (start 181.864 91.1225) (end 181.864 87.4395) (width 0.25) (layer F.Cu) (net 15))
 (segment (start 183.3245 92.583) (end 181.864 91.1225) (width 0.25) (layer F.Cu) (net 15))
 (segment (start 183.3245 103.124) (end 183.3245 92.583) (width 0.25) (layer F.Cu) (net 15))
 (segment (start 179.705 106.7435) (end 183.3245 103.124) (width 0.25) (layer F.Cu) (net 15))
 (segment (start 179.705 109.22) (end 174.625 104.14) (width 0.25) (layer F.Cu) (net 15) (status 80000))
 (segment (start 187.325 114.3) (end 182.245 109.22) (width 0.25) (layer B.Cu) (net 15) (status 80000))
 (segment (start 182.245 109.22) (end 179.705 109.22) (width 0.25) (layer B.Cu) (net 15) (status 80000))
 (segment (start 179.705 109.22) (end 180.975 110.49) (width 0.25) (layer F.Cu) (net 15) (status 80000))
 (segment (start 180.975 110.49) (end 180.975 120.65) (width 0.25) (layer F.Cu) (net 15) (status 80000))
 (segment (start 180.975 120.65) (end 179.705 121.92) (width 0.25) (layer F.Cu) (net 15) (status 80000)))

